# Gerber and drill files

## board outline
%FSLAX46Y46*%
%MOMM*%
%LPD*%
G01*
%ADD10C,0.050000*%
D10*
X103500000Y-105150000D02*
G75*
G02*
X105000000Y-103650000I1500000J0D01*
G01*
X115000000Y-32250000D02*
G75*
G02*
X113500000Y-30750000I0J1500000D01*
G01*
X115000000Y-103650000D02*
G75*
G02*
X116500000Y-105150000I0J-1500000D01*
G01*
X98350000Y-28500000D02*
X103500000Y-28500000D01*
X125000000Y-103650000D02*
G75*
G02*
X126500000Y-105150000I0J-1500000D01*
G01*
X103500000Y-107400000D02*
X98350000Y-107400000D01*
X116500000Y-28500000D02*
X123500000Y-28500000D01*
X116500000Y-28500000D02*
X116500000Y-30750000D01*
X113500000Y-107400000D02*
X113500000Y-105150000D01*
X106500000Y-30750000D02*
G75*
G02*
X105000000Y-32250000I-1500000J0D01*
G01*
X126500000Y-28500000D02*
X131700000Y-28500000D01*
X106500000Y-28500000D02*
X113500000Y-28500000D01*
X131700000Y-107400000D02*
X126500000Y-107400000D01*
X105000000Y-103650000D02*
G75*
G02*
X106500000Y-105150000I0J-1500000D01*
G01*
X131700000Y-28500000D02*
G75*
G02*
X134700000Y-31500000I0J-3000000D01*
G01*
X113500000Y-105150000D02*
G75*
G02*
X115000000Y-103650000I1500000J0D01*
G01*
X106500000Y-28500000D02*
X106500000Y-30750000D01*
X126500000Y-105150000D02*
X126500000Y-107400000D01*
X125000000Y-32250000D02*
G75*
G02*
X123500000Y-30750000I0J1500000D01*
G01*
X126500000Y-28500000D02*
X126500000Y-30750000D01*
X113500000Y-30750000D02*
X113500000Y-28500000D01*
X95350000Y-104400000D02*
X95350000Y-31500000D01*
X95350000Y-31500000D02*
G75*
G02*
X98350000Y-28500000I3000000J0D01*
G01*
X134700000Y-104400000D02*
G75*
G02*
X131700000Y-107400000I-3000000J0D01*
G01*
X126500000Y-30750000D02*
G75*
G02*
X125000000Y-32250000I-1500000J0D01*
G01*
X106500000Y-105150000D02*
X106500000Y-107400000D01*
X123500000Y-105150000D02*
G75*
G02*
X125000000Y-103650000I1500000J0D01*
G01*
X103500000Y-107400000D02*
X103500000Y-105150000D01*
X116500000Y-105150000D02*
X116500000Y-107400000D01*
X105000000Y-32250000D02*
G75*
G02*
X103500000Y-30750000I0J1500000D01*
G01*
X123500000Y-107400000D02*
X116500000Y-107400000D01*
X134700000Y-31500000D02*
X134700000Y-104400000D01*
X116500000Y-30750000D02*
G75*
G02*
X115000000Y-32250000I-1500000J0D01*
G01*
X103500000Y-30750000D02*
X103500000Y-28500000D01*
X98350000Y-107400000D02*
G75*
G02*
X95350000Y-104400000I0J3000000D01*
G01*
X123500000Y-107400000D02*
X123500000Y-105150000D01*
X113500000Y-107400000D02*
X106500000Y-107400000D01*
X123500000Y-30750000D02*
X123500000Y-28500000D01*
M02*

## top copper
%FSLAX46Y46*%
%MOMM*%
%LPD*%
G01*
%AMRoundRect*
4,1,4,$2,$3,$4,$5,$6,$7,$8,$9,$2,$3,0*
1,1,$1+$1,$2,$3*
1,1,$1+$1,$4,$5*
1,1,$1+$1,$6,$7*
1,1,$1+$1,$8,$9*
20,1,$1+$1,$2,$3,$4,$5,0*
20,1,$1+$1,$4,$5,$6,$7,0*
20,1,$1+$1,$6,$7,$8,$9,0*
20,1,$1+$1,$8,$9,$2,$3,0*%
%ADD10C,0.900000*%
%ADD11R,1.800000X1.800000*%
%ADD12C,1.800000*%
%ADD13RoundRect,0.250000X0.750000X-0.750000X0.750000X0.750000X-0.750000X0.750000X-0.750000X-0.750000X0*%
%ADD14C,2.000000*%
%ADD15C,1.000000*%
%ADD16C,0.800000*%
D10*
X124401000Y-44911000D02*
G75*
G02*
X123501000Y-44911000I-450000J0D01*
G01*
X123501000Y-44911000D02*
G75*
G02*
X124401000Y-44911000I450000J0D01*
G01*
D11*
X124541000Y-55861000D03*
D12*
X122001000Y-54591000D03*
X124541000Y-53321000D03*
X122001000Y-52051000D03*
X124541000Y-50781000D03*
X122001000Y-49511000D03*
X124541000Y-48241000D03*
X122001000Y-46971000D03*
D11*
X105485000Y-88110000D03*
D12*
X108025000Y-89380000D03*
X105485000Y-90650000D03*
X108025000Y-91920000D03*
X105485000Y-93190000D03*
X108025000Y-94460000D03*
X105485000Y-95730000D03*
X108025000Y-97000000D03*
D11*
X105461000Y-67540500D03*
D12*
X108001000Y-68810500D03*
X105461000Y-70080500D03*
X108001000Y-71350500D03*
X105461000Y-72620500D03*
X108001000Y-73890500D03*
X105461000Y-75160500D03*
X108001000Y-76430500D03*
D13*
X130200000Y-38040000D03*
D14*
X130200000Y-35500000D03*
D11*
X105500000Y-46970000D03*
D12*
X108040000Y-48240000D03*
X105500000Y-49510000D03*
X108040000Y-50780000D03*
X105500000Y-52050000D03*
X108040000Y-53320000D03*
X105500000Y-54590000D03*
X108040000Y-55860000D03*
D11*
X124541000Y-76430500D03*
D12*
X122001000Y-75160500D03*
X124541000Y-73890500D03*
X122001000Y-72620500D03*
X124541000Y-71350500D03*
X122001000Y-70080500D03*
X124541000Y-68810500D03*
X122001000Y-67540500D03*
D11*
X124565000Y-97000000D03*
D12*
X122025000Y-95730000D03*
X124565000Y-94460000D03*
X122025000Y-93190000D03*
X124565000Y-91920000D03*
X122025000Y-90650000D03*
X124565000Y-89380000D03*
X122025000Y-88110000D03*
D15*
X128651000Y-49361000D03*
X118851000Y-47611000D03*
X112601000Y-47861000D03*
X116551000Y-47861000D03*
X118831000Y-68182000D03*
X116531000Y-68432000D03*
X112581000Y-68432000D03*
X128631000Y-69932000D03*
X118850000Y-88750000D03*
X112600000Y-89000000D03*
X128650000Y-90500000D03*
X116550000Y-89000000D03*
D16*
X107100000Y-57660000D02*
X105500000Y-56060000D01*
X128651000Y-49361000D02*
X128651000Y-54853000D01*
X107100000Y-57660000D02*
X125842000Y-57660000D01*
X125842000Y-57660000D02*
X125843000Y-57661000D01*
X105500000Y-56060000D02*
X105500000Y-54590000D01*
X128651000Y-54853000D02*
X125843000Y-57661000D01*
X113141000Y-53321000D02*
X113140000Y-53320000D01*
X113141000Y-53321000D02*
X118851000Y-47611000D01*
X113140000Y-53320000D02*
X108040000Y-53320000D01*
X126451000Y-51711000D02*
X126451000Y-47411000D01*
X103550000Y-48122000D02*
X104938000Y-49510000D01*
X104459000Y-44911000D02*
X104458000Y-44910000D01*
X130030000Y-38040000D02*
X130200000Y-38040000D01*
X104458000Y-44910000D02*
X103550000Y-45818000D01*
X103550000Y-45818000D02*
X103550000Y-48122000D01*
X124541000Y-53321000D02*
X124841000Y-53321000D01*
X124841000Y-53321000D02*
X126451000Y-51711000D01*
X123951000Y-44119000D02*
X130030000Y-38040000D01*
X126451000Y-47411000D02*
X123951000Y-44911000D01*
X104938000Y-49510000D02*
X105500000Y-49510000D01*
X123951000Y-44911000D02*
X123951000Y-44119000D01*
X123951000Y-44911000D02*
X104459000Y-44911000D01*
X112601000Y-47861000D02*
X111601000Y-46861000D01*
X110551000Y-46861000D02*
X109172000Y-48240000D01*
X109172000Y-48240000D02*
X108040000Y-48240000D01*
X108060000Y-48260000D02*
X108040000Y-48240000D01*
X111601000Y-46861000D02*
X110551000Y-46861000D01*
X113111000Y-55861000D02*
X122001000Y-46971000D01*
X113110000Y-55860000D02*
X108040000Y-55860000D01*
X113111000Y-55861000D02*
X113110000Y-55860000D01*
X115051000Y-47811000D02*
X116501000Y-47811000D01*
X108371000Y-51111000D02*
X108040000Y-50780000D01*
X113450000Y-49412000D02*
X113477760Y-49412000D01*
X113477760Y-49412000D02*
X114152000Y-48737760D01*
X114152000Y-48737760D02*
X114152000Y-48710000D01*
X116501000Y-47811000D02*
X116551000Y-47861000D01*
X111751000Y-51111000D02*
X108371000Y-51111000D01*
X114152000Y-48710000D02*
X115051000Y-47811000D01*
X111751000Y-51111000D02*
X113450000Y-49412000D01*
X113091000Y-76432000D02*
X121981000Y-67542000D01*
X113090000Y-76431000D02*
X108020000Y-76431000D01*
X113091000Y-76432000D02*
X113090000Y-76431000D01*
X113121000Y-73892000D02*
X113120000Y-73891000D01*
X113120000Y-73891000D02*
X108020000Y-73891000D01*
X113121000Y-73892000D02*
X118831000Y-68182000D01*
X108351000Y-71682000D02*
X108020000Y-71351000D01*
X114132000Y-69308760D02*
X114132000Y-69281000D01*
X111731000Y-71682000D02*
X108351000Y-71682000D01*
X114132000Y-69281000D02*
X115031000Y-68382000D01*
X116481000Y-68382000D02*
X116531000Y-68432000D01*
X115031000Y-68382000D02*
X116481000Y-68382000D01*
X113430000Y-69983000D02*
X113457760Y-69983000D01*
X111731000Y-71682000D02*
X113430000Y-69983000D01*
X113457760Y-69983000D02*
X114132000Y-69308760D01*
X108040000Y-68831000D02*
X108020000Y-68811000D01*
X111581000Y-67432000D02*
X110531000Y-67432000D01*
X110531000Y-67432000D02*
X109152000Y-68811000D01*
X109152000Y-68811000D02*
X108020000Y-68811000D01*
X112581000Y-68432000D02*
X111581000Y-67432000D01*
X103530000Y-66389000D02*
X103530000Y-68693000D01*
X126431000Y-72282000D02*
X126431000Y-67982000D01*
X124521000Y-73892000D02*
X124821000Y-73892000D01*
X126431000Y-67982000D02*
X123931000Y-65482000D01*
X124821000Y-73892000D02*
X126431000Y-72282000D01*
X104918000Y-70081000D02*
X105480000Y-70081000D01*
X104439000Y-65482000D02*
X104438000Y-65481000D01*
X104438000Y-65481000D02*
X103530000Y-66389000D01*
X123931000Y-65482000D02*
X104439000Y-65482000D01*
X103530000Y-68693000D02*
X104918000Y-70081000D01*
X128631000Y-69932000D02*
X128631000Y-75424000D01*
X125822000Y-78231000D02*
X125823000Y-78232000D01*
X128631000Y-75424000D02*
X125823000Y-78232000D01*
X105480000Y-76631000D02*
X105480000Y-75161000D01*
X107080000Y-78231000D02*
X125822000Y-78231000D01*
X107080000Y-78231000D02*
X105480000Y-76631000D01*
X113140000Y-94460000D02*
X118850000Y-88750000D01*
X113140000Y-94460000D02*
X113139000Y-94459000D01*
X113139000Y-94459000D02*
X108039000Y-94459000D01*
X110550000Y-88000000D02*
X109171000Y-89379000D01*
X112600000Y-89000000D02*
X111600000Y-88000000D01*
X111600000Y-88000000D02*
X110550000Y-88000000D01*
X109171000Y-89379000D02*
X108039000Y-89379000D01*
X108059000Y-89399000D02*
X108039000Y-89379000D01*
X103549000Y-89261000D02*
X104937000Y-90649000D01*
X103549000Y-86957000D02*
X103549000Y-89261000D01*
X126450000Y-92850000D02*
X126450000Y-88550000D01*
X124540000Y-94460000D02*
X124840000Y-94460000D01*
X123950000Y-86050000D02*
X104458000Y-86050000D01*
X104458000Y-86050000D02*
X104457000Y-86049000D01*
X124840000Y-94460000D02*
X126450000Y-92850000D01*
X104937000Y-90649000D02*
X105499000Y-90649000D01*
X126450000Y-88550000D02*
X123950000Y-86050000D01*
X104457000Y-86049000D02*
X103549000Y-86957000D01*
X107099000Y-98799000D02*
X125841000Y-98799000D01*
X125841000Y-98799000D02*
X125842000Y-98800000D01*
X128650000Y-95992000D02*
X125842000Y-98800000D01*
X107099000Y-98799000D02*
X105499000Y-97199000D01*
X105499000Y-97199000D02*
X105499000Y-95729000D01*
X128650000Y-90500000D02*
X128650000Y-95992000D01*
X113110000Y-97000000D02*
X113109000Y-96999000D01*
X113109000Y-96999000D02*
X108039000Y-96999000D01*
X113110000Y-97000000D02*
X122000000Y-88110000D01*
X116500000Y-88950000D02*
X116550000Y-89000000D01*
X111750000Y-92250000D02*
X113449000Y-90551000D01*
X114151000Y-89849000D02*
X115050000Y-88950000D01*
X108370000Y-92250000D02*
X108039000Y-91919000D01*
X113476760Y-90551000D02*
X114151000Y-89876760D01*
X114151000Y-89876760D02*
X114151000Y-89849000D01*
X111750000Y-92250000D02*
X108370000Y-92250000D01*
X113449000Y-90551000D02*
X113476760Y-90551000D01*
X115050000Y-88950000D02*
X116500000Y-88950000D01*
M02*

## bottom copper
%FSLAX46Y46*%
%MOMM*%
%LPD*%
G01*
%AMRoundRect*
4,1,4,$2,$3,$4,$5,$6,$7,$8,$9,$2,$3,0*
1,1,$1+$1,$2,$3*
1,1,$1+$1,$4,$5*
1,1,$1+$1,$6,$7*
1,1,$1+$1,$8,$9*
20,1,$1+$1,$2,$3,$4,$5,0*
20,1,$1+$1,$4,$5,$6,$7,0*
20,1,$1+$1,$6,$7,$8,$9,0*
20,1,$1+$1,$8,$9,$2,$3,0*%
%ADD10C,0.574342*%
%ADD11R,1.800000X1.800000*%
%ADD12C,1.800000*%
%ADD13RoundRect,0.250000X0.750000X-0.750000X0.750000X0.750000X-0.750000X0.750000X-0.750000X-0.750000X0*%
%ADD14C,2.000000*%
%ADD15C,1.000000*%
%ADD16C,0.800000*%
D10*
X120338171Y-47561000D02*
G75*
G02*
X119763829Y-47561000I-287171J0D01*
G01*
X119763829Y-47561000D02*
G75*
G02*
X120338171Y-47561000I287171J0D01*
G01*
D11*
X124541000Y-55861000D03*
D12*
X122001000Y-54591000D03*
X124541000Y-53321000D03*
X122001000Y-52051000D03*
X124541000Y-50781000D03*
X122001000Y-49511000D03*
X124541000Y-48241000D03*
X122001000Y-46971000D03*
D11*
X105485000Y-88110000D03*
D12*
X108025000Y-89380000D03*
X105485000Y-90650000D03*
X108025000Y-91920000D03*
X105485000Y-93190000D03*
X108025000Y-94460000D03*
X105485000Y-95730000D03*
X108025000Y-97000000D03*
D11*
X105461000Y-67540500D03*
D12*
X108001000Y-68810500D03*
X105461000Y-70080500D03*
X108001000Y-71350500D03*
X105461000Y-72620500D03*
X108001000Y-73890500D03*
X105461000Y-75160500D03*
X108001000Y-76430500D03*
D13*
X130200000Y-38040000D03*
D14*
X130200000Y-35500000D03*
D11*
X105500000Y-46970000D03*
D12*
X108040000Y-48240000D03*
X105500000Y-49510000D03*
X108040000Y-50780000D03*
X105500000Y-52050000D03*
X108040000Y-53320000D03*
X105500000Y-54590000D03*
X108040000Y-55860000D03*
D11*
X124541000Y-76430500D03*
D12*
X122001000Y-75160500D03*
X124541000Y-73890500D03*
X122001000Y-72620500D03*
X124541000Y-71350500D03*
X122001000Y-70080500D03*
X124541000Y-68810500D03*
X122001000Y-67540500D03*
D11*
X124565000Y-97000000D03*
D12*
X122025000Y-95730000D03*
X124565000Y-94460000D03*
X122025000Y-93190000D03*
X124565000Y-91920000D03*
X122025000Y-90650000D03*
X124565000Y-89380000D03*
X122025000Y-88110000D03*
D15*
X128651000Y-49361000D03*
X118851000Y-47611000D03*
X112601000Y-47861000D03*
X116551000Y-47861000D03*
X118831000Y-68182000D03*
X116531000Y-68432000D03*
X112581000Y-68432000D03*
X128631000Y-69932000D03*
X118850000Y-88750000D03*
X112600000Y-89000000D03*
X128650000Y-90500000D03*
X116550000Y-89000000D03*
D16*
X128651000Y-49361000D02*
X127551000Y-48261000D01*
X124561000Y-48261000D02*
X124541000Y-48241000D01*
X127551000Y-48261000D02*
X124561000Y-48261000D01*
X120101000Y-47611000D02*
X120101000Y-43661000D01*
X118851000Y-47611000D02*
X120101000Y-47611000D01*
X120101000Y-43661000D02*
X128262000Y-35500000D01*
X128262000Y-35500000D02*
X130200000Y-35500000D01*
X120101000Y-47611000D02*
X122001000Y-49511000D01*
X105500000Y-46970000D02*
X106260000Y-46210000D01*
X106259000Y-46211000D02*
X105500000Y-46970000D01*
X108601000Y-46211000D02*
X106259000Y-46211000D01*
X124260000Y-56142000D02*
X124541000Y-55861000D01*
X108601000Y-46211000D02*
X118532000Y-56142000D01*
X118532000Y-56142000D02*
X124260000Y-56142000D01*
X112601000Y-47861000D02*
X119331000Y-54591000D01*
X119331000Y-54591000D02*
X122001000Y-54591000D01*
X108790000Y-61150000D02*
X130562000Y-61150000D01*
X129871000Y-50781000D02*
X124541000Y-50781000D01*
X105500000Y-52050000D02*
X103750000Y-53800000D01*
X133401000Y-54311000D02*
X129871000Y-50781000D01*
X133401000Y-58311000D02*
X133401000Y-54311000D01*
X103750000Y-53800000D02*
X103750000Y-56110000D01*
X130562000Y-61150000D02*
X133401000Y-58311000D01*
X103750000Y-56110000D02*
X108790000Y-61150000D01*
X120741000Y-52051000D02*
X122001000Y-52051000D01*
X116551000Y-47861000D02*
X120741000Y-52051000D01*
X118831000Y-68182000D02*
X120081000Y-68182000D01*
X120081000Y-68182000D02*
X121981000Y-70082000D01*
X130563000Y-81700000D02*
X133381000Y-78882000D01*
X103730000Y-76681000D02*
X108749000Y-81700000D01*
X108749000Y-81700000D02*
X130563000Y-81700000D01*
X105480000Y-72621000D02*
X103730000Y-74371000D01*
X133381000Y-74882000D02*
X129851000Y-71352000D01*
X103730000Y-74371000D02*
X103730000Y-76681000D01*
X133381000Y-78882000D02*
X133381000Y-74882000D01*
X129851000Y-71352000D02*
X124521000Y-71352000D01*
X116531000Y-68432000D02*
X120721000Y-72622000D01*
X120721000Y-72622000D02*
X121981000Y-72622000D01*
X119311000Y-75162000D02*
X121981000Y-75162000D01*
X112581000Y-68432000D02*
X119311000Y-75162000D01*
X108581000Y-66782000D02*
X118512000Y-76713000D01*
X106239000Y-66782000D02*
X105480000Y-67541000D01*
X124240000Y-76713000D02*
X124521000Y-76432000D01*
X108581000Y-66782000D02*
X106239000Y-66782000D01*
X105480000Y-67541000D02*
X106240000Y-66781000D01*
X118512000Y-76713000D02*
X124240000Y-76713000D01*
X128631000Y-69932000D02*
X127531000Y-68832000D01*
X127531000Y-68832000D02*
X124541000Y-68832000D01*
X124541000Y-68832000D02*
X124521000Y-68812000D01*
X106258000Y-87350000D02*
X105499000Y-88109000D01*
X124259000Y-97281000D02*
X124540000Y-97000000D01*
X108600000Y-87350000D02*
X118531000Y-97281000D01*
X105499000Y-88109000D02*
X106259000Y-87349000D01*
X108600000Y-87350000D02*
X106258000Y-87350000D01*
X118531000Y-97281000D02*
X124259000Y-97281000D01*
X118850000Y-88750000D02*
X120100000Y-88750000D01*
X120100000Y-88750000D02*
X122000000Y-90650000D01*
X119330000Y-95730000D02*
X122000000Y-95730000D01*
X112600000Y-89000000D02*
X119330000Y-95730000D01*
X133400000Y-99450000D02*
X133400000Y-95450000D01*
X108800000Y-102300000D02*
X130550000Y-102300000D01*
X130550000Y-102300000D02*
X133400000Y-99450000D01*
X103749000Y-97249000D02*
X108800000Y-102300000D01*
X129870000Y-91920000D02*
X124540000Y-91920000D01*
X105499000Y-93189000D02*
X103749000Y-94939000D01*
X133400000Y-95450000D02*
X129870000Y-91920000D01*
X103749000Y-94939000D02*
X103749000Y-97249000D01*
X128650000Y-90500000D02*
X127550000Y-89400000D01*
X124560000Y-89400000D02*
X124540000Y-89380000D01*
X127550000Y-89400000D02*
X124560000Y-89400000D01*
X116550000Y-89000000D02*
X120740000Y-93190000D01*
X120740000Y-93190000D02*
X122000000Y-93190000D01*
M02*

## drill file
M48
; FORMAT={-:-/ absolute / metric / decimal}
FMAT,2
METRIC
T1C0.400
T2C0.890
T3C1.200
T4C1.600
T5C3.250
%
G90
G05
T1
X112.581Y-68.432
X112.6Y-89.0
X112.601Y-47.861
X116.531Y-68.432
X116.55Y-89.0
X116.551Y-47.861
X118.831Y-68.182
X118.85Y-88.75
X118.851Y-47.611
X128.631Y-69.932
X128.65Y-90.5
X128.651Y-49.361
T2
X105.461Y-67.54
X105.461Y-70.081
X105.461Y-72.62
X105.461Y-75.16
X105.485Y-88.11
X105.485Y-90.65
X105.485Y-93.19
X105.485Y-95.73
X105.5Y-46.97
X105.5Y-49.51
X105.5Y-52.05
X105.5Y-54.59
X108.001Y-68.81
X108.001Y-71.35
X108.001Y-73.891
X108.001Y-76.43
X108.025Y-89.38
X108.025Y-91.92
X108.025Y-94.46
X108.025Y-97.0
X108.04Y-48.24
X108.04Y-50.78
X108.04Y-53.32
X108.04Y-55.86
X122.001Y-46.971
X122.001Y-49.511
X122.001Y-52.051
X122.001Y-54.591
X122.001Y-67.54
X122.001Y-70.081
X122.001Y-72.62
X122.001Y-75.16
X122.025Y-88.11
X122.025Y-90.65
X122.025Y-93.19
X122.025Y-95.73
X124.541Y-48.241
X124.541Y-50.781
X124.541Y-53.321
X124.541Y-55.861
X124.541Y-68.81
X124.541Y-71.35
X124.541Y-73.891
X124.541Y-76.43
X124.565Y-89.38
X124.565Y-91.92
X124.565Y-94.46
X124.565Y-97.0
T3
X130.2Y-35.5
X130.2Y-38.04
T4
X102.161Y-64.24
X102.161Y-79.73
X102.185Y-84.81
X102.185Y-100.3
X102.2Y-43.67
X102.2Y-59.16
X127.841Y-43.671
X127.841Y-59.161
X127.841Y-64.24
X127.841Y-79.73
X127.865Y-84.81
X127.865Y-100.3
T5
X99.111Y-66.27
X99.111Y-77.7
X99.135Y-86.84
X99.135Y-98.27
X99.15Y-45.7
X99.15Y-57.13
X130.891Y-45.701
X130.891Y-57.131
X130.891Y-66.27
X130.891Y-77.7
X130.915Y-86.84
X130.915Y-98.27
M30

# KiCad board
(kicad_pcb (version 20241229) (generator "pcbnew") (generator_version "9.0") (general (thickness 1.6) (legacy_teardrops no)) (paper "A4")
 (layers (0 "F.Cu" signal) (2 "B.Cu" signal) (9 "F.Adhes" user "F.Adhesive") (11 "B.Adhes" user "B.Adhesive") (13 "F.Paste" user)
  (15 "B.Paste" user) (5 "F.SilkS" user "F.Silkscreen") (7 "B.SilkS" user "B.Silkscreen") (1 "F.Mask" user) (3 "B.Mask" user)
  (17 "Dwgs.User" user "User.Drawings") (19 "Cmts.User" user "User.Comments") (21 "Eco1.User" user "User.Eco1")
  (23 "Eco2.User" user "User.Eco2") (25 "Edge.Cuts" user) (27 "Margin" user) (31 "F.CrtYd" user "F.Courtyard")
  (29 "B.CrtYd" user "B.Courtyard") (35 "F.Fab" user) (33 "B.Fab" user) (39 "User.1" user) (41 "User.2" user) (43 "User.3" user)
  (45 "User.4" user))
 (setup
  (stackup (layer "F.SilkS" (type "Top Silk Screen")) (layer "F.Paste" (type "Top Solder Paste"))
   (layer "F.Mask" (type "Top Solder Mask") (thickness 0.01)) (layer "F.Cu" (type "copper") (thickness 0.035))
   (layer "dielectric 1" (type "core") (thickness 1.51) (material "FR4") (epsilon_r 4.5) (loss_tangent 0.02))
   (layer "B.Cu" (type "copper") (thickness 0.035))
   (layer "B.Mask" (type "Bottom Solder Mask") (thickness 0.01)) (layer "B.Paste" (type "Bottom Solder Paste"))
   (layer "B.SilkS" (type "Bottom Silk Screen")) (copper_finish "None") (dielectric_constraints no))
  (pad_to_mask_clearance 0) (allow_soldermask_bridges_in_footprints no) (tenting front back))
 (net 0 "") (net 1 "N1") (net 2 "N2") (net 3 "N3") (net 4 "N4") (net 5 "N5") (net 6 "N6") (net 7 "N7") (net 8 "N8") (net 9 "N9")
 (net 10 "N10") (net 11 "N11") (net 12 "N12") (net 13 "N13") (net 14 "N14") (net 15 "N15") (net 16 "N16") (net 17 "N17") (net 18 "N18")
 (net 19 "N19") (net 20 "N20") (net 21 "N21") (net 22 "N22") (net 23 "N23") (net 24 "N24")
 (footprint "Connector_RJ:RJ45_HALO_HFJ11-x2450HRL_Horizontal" (layer "F.Cu") (at 124.541 55.861 90)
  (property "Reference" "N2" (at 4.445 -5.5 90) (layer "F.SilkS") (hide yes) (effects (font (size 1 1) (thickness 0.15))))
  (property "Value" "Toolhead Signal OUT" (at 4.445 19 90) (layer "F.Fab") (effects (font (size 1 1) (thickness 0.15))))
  (pad "" np_thru_hole circle (at -3.3 3.3 90) (size 3 3) (drill 1.6) (layers "*.Mask"))
  (pad "" np_thru_hole circle (at -1.27 6.35 90) (size 3.25 3.25) (drill 3.25) (layers "*.Cu" "*.Mask"))
  (pad "" np_thru_hole circle (at 10.16 6.35 90) (size 3.25 3.25) (drill 3.25) (layers "*.Cu" "*.Mask"))
  (pad "" np_thru_hole circle (at 12.19 3.3 90) (size 3 3) (drill 1.6) (layers "*.Mask"))
  (pad "1" thru_hole rect (at 0 0 90) (size 1.8 1.8) (drill 0.89) (layers "*.Cu" "*.Mask") (remove_unused_layers no) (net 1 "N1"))
  (pad "2" thru_hole circle (at 1.27 -2.54 90) (size 1.8 1.8) (drill 0.89) (layers "*.Cu" "*.Mask") (remove_unused_layers no) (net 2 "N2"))
  (pad "3" thru_hole circle (at 2.54 0 90) (size 1.8 1.8) (drill 0.89) (layers "*.Cu" "*.Mask") (remove_unused_layers no) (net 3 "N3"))
  (pad "4" thru_hole circle (at 3.81 -2.54 90) (size 1.8 1.8) (drill 0.89) (layers "*.Cu" "*.Mask") (remove_unused_layers no) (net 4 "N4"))
  (pad "5" thru_hole circle (at 5.08 0 90) (size 1.8 1.8) (drill 0.89) (layers "*.Cu" "*.Mask") (remove_unused_layers no) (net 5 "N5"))
  (pad "6" thru_hole circle (at 6.35 -2.54 90) (size 1.8 1.8) (drill 0.89) (layers "*.Cu" "*.Mask") (remove_unused_layers no) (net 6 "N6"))
  (pad "7" thru_hole circle (at 7.62 0 90) (size 1.8 1.8) (drill 0.89) (layers "*.Cu" "*.Mask") (remove_unused_layers no) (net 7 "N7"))
  (pad "8" thru_hole circle (at 8.89 -2.54 90) (size 1.8 1.8) (drill 0.89) (layers "*.Cu" "*.Mask") (remove_unused_layers no) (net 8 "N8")))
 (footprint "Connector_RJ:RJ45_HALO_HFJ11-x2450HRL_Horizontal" (layer "F.Cu") (at 105.485 88.11 -90)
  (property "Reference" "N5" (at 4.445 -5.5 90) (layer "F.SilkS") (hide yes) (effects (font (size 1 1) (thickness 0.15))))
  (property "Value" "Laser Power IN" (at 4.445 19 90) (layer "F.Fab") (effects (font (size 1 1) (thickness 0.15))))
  (pad "" np_thru_hole circle (at -3.3 3.3 270) (size 3 3) (drill 1.6) (layers "*.Mask"))
  (pad "" np_thru_hole circle (at -1.27 6.35 270) (size 3.25 3.25) (drill 3.25) (layers "*.Cu" "*.Mask"))
  (pad "" np_thru_hole circle (at 10.16 6.35 270) (size 3.25 3.25) (drill 3.25) (layers "*.Cu" "*.Mask"))
  (pad "" np_thru_hole circle (at 12.19 3.3 270) (size 3 3) (drill 1.6) (layers "*.Mask"))
  (pad "1" thru_hole rect (at 0 0 270) (size 1.8 1.8) (drill 0.89) (layers "*.Cu" "*.Mask") (remove_unused_layers no) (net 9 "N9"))
  (pad "2" thru_hole circle (at 1.27 -2.54 270) (size 1.8 1.8) (drill 0.89) (layers "*.Cu" "*.Mask") (remove_unused_layers no)
   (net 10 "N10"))
  (pad "3" thru_hole circle (at 2.54 0 270) (size 1.8 1.8) (drill 0.89) (layers "*.Cu" "*.Mask") (remove_unused_layers no) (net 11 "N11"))
  (pad "4" thru_hole circle (at 3.81 -2.54 270) (size 1.8 1.8) (drill 0.89) (layers "*.Cu" "*.Mask") (remove_unused_layers no)
   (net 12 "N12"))
  (pad "5" thru_hole circle (at 5.08 0 270) (size 1.8 1.8) (drill 0.89) (layers "*.Cu" "*.Mask") (remove_unused_layers no) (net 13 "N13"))
  (pad "6" thru_hole circle (at 6.35 -2.54 270) (size 1.8 1.8) (drill 0.89) (layers "*.Cu" "*.Mask") (remove_unused_layers no)
   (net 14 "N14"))
  (pad "7" thru_hole circle (at 7.62 0 270) (size 1.8 1.8) (drill 0.89) (layers "*.Cu" "*.Mask") (remove_unused_layers no) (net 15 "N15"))
  (pad "8" thru_hole circle (at 8.89 -2.54 270) (size 1.8 1.8) (drill 0.89) (layers "*.Cu" "*.Mask") (remove_unused_layers no)
   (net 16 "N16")))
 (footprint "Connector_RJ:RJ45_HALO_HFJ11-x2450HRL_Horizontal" (layer "F.Cu") (at 105.461 67.5405 -90)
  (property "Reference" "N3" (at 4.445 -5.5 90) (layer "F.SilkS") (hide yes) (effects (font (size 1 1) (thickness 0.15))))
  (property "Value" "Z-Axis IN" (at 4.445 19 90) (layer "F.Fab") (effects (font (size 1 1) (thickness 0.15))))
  (pad "" np_thru_hole circle (at -3.3 3.3 270) (size 3 3) (drill 1.6) (layers "*.Mask"))
  (pad "" np_thru_hole circle (at -1.27 6.35 270) (size 3.25 3.25) (drill 3.25) (layers "*.Cu" "*.Mask"))
  (pad "" np_thru_hole circle (at 10.16 6.35 270) (size 3.25 3.25) (drill 3.25) (layers "*.Cu" "*.Mask"))
  (pad "" np_thru_hole circle (at 12.19 3.3 270) (size 3 3) (drill 1.6) (layers "*.Mask"))
  (pad "1" thru_hole rect (at 0 0 270) (size 1.8 1.8) (drill 0.89) (layers "*.Cu" "*.Mask") (remove_unused_layers no) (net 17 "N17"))
  (pad "2" thru_hole circle (at 1.27 -2.54 270) (size 1.8 1.8) (drill 0.89) (layers "*.Cu" "*.Mask") (remove_unused_layers no)
   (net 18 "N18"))
  (pad "3" thru_hole circle (at 2.54 0 270) (size 1.8 1.8) (drill 0.89) (layers "*.Cu" "*.Mask") (remove_unused_layers no) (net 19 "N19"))
  (pad "4" thru_hole circle (at 3.81 -2.54 270) (size 1.8 1.8) (drill 0.89) (layers "*.Cu" "*.Mask") (remove_unused_layers no)
   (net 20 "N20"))
  (pad "5" thru_hole circle (at 5.08 0 270) (size 1.8 1.8) (drill 0.89) (layers "*.Cu" "*.Mask") (remove_unused_layers no) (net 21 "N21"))
  (pad "6" thru_hole circle (at 6.35 -2.54 270) (size 1.8 1.8) (drill 0.89) (layers "*.Cu" "*.Mask") (remove_unused_layers no)
   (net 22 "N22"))
  (pad "7" thru_hole circle (at 7.62 0 270) (size 1.8 1.8) (drill 0.89) (layers "*.Cu" "*.Mask") (remove_unused_layers no) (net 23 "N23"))
  (pad "8" thru_hole circle (at 8.89 -2.54 270) (size 1.8 1.8) (drill 0.89) (layers "*.Cu" "*.Mask") (remove_unused_layers no)
   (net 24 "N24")))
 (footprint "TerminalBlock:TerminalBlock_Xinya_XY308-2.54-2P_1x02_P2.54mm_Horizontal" (layer "F.Cu") (at 130.2 38.04 90)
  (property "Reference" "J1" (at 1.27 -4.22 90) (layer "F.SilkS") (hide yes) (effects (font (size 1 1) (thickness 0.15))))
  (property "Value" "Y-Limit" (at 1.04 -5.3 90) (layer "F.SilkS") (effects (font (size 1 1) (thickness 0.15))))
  (pad "1" thru_hole roundrect (at 0 0 90) (size 2 2) (drill 1.2) (layers "*.Cu" "*.Mask") (remove_unused_layers no)
   (roundrect_rratio 0.125) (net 3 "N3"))
  (pad "2" thru_hole circle (at 2.54 0 90) (size 2 2) (drill 1.2) (layers "*.Cu" "*.Mask") (remove_unused_layers no) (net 6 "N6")))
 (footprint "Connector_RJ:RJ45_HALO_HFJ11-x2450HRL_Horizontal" (layer "F.Cu") (at 105.5 46.97 -90)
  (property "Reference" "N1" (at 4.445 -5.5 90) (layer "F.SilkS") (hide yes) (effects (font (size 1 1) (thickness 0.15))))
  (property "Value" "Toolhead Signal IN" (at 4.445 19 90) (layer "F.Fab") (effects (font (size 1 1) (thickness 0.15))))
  (pad "" np_thru_hole circle (at -3.3 3.3 270) (size 3 3) (drill 1.6) (layers "*.Mask"))
  (pad "" np_thru_hole circle (at -1.27 6.35 270) (size 3.25 3.25) (drill 3.25) (layers "*.Cu" "*.Mask"))
  (pad "" np_thru_hole circle (at 10.16 6.35 270) (size 3.25 3.25) (drill 3.25) (layers "*.Cu" "*.Mask"))
  (pad "" np_thru_hole circle (at 12.19 3.3 270) (size 3 3) (drill 1.6) (layers "*.Mask"))
  (pad "1" thru_hole rect (at 0 0 270) (size 1.8 1.8) (drill 0.89) (layers "*.Cu" "*.Mask") (remove_unused_layers no) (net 1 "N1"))
  (pad "2" thru_hole circle (at 1.27 -2.54 270) (size 1.8 1.8) (drill 0.89) (layers "*.Cu" "*.Mask") (remove_unused_layers no) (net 2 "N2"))
  (pad "3" thru_hole circle (at 2.54 0 270) (size 1.8 1.8) (drill 0.89) (layers "*.Cu" "*.Mask") (remove_unused_layers no) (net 3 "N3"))
  (pad "4" thru_hole circle (at 3.81 -2.54 270) (size 1.8 1.8) (drill 0.89) (layers "*.Cu" "*.Mask") (remove_unused_layers no) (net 4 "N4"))
  (pad "5" thru_hole circle (at 5.08 0 270) (size 1.8 1.8) (drill 0.89) (layers "*.Cu" "*.Mask") (remove_unused_layers no) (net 5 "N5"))
  (pad "6" thru_hole circle (at 6.35 -2.54 270) (size 1.8 1.8) (drill 0.89) (layers "*.Cu" "*.Mask") (remove_unused_layers no) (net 6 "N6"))
  (pad "7" thru_hole circle (at 7.62 0 270) (size 1.8 1.8) (drill 0.89) (layers "*.Cu" "*.Mask") (remove_unused_layers no) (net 7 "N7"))
  (pad "8" thru_hole circle (at 8.89 -2.54 270) (size 1.8 1.8) (drill 0.89) (layers "*.Cu" "*.Mask") (remove_unused_layers no) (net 8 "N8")))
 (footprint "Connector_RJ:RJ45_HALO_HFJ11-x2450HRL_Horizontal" (layer "F.Cu") (at 124.541 76.4305 90)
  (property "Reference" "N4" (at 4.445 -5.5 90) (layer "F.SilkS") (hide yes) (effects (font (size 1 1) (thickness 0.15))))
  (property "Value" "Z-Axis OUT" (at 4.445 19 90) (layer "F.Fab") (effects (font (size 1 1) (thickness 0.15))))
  (pad "" np_thru_hole circle (at -3.3 3.3 90) (size 3 3) (drill 1.6) (layers "*.Mask"))
  (pad "" np_thru_hole circle (at -1.27 6.35 90) (size 3.25 3.25) (drill 3.25) (layers "*.Cu" "*.Mask"))
  (pad "" np_thru_hole circle (at 10.16 6.35 90) (size 3.25 3.25) (drill 3.25) (layers "*.Cu" "*.Mask"))
  (pad "" np_thru_hole circle (at 12.19 3.3 90) (size 3 3) (drill 1.6) (layers "*.Mask"))
  (pad "1" thru_hole rect (at 0 0 90) (size 1.8 1.8) (drill 0.89) (layers "*.Cu" "*.Mask") (remove_unused_layers no) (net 17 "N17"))
  (pad "2" thru_hole circle (at 1.27 -2.54 90) (size 1.8 1.8) (drill 0.89) (layers "*.Cu" "*.Mask") (remove_unused_layers no) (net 18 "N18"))
  (pad "3" thru_hole circle (at 2.54 0 90) (size 1.8 1.8) (drill 0.89) (layers "*.Cu" "*.Mask") (remove_unused_layers no) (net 19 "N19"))
  (pad "4" thru_hole circle (at 3.81 -2.54 90) (size 1.8 1.8) (drill 0.89) (layers "*.Cu" "*.Mask") (remove_unused_layers no) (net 20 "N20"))
  (pad "5" thru_hole circle (at 5.08 0 90) (size 1.8 1.8) (drill 0.89) (layers "*.Cu" "*.Mask") (remove_unused_layers no) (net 21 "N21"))
  (pad "6" thru_hole circle (at 6.35 -2.54 90) (size 1.8 1.8) (drill 0.89) (layers "*.Cu" "*.Mask") (remove_unused_layers no) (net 22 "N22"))
  (pad "7" thru_hole circle (at 7.62 0 90) (size 1.8 1.8) (drill 0.89) (layers "*.Cu" "*.Mask") (remove_unused_layers no) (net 23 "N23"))
  (pad "8" thru_hole circle (at 8.89 -2.54 90) (size 1.8 1.8) (drill 0.89) (layers "*.Cu" "*.Mask") (remove_unused_layers no) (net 24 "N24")))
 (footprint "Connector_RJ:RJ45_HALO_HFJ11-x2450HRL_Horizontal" (layer "F.Cu") (at 124.565 97 90)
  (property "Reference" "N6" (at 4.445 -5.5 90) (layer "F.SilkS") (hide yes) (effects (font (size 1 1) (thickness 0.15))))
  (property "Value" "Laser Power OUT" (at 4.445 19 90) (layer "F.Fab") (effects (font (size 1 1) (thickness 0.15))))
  (pad "" np_thru_hole circle (at -3.3 3.3 90) (size 3 3) (drill 1.6) (layers "*.Mask"))
  (pad "" np_thru_hole circle (at -1.27 6.35 90) (size 3.25 3.25) (drill 3.25) (layers "*.Cu" "*.Mask"))
  (pad "" np_thru_hole circle (at 10.16 6.35 90) (size 3.25 3.25) (drill 3.25) (layers "*.Cu" "*.Mask"))
  (pad "" np_thru_hole circle (at 12.19 3.3 90) (size 3 3) (drill 1.6) (layers "*.Mask"))
  (pad "1" thru_hole rect (at 0 0 90) (size 1.8 1.8) (drill 0.89) (layers "*.Cu" "*.Mask") (remove_unused_layers no) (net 9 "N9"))
  (pad "2" thru_hole circle (at 1.27 -2.54 90) (size 1.8 1.8) (drill 0.89) (layers "*.Cu" "*.Mask") (remove_unused_layers no) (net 10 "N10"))
  (pad "3" thru_hole circle (at 2.54 0 90) (size 1.8 1.8) (drill 0.89) (layers "*.Cu" "*.Mask") (remove_unused_layers no) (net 11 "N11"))
  (pad "4" thru_hole circle (at 3.81 -2.54 90) (size 1.8 1.8) (drill 0.89) (layers "*.Cu" "*.Mask") (remove_unused_layers no) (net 12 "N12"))
  (pad "5" thru_hole circle (at 5.08 0 90) (size 1.8 1.8) (drill 0.89) (layers "*.Cu" "*.Mask") (remove_unused_layers no) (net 13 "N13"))
  (pad "6" thru_hole circle (at 6.35 -2.54 90) (size 1.8 1.8) (drill 0.89) (layers "*.Cu" "*.Mask") (remove_unused_layers no) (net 14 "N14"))
  (pad "7" thru_hole circle (at 7.62 0 90) (size 1.8 1.8) (drill 0.89) (layers "*.Cu" "*.Mask") (remove_unused_layers no) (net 15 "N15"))
  (pad "8" thru_hole circle (at 8.89 -2.54 90) (size 1.8 1.8) (drill 0.89) (layers "*.Cu" "*.Mask") (remove_unused_layers no) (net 16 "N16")))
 (gr_circle (center 123.951 44.911) (end 124.751 44.911) (stroke (width 0.2) (type solid)) (fill yes) (layer "F.Cu") (net 3))
 (gr_circle (center 120.051 47.561) (end 120.501 47.411) (stroke (width 0.2) (type solid)) (fill yes) (layer "B.Cu") (net 6))
 (gr_arc (start 103.5 105.15) (mid 103.93934 104.08934) (end 105 103.65) (stroke (width 0.05) (type default)) (layer "Edge.Cuts"))
 (gr_arc (start 115 32.25) (mid 113.93934 31.81066) (end 113.5 30.75) (stroke (width 0.05) (type default)) (layer "Edge.Cuts"))
 (gr_arc (start 115 103.65) (mid 116.06066 104.08934) (end 116.5 105.15) (stroke (width 0.05) (type default)) (layer "Edge.Cuts"))
 (gr_line (start 98.35 28.5) (end 103.5 28.5) (stroke (width 0.05) (type default)) (layer "Edge.Cuts"))
 (gr_arc (start 125 103.65) (mid 126.06066 104.08934) (end 126.5 105.15) (stroke (width 0.05) (type default)) (layer "Edge.Cuts"))
 (gr_line (start 103.5 107.4) (end 98.35 107.4) (stroke (width 0.05) (type default)) (layer "Edge.Cuts"))
 (gr_line (start 116.5 28.5) (end 123.5 28.5) (stroke (width 0.05) (type default)) (layer "Edge.Cuts"))
 (gr_line (start 116.5 28.5) (end 116.5 30.75) (stroke (width 0.05) (type solid)) (layer "Edge.Cuts"))
 (gr_line (start 113.5 107.4) (end 113.5 105.15) (stroke (width 0.05) (type solid)) (layer "Edge.Cuts"))
 (gr_arc (start 106.5 30.75) (mid 106.06066 31.81066) (end 105 32.25) (stroke (width 0.05) (type default)) (layer "Edge.Cuts"))
 (gr_line (start 126.5 28.5) (end 131.7 28.5) (stroke (width 0.05) (type default)) (layer "Edge.Cuts"))
 (gr_line (start 106.5 28.5) (end 113.5 28.5) (stroke (width 0.05) (type default)) (layer "Edge.Cuts"))
 (gr_line (start 131.7 107.4) (end 126.5 107.4) (stroke (width 0.05) (type default)) (layer "Edge.Cuts"))
 (gr_arc (start 105 103.65) (mid 106.06066 104.08934) (end 106.5 105.15) (stroke (width 0.05) (type default)) (layer "Edge.Cuts"))
 (gr_arc (start 131.7 28.5) (mid 133.82132 29.37868) (end 134.7 31.5) (stroke (width 0.05) (type default)) (layer "Edge.Cuts"))
 (gr_arc (start 113.5 105.15) (mid 113.93934 104.08934) (end 115 103.65) (stroke (width 0.05) (type default)) (layer "Edge.Cuts"))
 (gr_line (start 106.5 28.5) (end 106.5 30.75) (stroke (width 0.05) (type solid)) (layer "Edge.Cuts"))
 (gr_line (start 126.5 105.15) (end 126.5 107.4) (stroke (width 0.05) (type solid)) (layer "Edge.Cuts"))
 (gr_arc (start 125 32.25) (mid 123.93934 31.81066) (end 123.5 30.75) (stroke (width 0.05) (type default)) (layer "Edge.Cuts"))
 (gr_line (start 126.5 28.5) (end 126.5 30.75) (stroke (width 0.05) (type solid)) (layer "Edge.Cuts"))
 (gr_line (start 113.5 30.75) (end 113.5 28.5) (stroke (width 0.05) (type solid)) (layer "Edge.Cuts"))
 (gr_line (start 95.35 104.4) (end 95.35 31.5) (stroke (width 0.05) (type default)) (layer "Edge.Cuts"))
 (gr_arc (start 95.35 31.5) (mid 96.22868 29.37868) (end 98.35 28.5) (stroke (width 0.05) (type default)) (layer "Edge.Cuts"))
 (gr_arc (start 134.7 104.4) (mid 133.82132 106.52132) (end 131.7 107.4) (stroke (width 0.05) (type default)) (layer "Edge.Cuts"))
 (gr_arc (start 126.5 30.75) (mid 126.06066 31.81066) (end 125 32.25) (stroke (width 0.05) (type default)) (layer "Edge.Cuts"))
 (gr_line (start 106.5 105.15) (end 106.5 107.4) (stroke (width 0.05) (type solid)) (layer "Edge.Cuts"))
 (gr_arc (start 123.5 105.15) (mid 123.93934 104.08934) (end 125 103.65) (stroke (width 0.05) (type default)) (layer "Edge.Cuts"))
 (gr_line (start 103.5 107.4) (end 103.5 105.15) (stroke (width 0.05) (type solid)) (layer "Edge.Cuts"))
 (gr_line (start 116.5 105.15) (end 116.5 107.4) (stroke (width 0.05) (type solid)) (layer "Edge.Cuts"))
 (gr_arc (start 105 32.25) (mid 103.93934 31.81066) (end 103.5 30.75) (stroke (width 0.05) (type default)) (layer "Edge.Cuts"))
 (gr_line (start 123.5 107.4) (end 116.5 107.4) (stroke (width 0.05) (type default)) (layer "Edge.Cuts"))
 (gr_line (start 134.7 31.5) (end 134.7 104.4) (stroke (width 0.05) (type default)) (layer "Edge.Cuts"))
 (gr_arc (start 116.5 30.75) (mid 116.06066 31.81066) (end 115 32.25) (stroke (width 0.05) (type default)) (layer "Edge.Cuts"))
 (gr_line (start 103.5 30.75) (end 103.5 28.5) (stroke (width 0.05) (type solid)) (layer "Edge.Cuts"))
 (gr_arc (start 98.35 107.4) (mid 96.22868 106.52132) (end 95.35 104.4) (stroke (width 0.05) (type default)) (layer "Edge.Cuts"))
 (gr_line (start 123.5 107.4) (end 123.5 105.15) (stroke (width 0.05) (type solid)) (layer "Edge.Cuts"))
 (gr_line (start 113.5 107.4) (end 106.5 107.4) (stroke (width 0.05) (type default)) (layer "Edge.Cuts"))
 (gr_line (start 123.5 30.75) (end 123.5 28.5) (stroke (width 0.05) (type solid)) (layer "Edge.Cuts"))
 (segment (start 107.1 57.66) (end 105.5 56.06) (width 0.8) (layer "F.Cu") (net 7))
 (segment (start 128.651 49.361) (end 128.651 54.853) (width 0.8) (layer "F.Cu") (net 7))
 (segment (start 107.1 57.66) (end 125.842 57.66) (width 0.8) (layer "F.Cu") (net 7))
 (segment (start 125.842 57.66) (end 125.843 57.661) (width 0.8) (layer "F.Cu") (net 7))
 (segment (start 105.5 56.06) (end 105.5 54.59) (width 0.8) (layer "F.Cu") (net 7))
 (segment (start 128.651 54.853) (end 125.843 57.661) (width 0.8) (layer "F.Cu") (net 7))
 (via (at 128.651 49.361) (size 1) (drill 0.4) (layers "F.Cu" "B.Cu") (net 7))
 (segment (start 128.651 49.361) (end 127.551 48.261) (width 0.8) (layer "B.Cu") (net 7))
 (segment (start 124.561 48.261) (end 124.541 48.241) (width 0.8) (layer "B.Cu") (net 7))
 (segment (start 127.551 48.261) (end 124.561 48.261) (width 0.8) (layer "B.Cu") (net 7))
 (segment (start 113.141 53.321) (end 113.14 53.32) (width 0.8) (layer "F.Cu") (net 6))
 (segment (start 113.141 53.321) (end 118.851 47.611) (width 0.8) (layer "F.Cu") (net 6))
 (segment (start 113.14 53.32) (end 108.04 53.32) (width 0.8) (layer "F.Cu") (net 6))
 (via (at 118.851 47.611) (size 1) (drill 0.4) (layers "F.Cu" "B.Cu") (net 6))
 (segment (start 120.101 47.611) (end 120.101 43.661) (width 0.8) (layer "B.Cu") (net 6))
 (segment (start 118.851 47.611) (end 120.101 47.611) (width 0.8) (layer "B.Cu") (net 6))
 (segment (start 120.101 43.661) (end 128.262 35.5) (width 0.8) (layer "B.Cu") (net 6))
 (segment (start 128.262 35.5) (end 130.2 35.5) (width 0.8) (layer "B.Cu") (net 6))
 (segment (start 120.101 47.611) (end 122.001 49.511) (width 0.8) (layer "B.Cu") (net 6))
 (segment (start 126.451 51.711) (end 126.451 47.411) (width 0.8) (layer "F.Cu") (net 3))
 (segment (start 103.55 48.122) (end 104.938 49.51) (width 0.8) (layer "F.Cu") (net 3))
 (segment (start 104.459 44.911) (end 104.458 44.91) (width 0.8) (layer "F.Cu") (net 3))
 (segment (start 130.03 38.04) (end 130.2 38.04) (width 0.8) (layer "F.Cu") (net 3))
 (segment (start 104.458 44.91) (end 103.55 45.818) (width 0.8) (layer "F.Cu") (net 3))
 (segment (start 103.55 45.818) (end 103.55 48.122) (width 0.8) (layer "F.Cu") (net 3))
 (segment (start 124.541 53.321) (end 124.841 53.321) (width 0.8) (layer "F.Cu") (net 3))
 (segment (start 124.841 53.321) (end 126.451 51.711) (width 0.8) (layer "F.Cu") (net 3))
 (segment (start 123.951 44.119) (end 130.03 38.04) (width 0.8) (layer "F.Cu") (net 3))
 (segment (start 126.451 47.411) (end 123.951 44.911) (width 0.8) (layer "F.Cu") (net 3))
 (segment (start 104.938 49.51) (end 105.5 49.51) (width 0.8) (layer "F.Cu") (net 3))
 (segment (start 123.951 44.911) (end 123.951 44.119) (width 0.8) (layer "F.Cu") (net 3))
 (segment (start 123.951 44.911) (end 104.459 44.911) (width 0.8) (layer "F.Cu") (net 3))
 (segment (start 105.5 46.97) (end 106.26 46.21) (width 0.8) (layer "B.Cu") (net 1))
 (segment (start 106.259 46.211) (end 105.5 46.97) (width 0.8) (layer "B.Cu") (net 1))
 (segment (start 108.601 46.211) (end 106.259 46.211) (width 0.8) (layer "B.Cu") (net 1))
 (segment (start 124.26 56.142) (end 124.541 55.861) (width 0.8) (layer "B.Cu") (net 1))
 (segment (start 108.601 46.211) (end 118.532 56.142) (width 0.8) (layer "B.Cu") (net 1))
 (segment (start 118.532 56.142) (end 124.26 56.142) (width 0.8) (layer "B.Cu") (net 1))
 (segment (start 112.601 47.861) (end 111.601 46.861) (width 0.8) (layer "F.Cu") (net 2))
 (segment (start 110.551 46.861) (end 109.172 48.24) (width 0.8) (layer "F.Cu") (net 2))
 (segment (start 109.172 48.24) (end 108.04 48.24) (width 0.8) (layer "F.Cu") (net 2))
 (segment (start 108.06 48.26) (end 108.04 48.24) (width 0.8) (layer "F.Cu") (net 2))
 (segment (start 111.601 46.861) (end 110.551 46.861) (width 0.8) (layer "F.Cu") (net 2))
 (via (at 112.601 47.861) (size 1) (drill 0.4) (layers "F.Cu" "B.Cu") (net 2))
 (segment (start 112.601 47.861) (end 119.331 54.591) (width 0.8) (layer "B.Cu") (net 2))
 (segment (start 119.331 54.591) (end 122.001 54.591) (width 0.8) (layer "B.Cu") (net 2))
 (segment (start 108.79 61.15) (end 130.562 61.15) (width 0.8) (layer "B.Cu") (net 5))
 (segment (start 129.871 50.781) (end 124.541 50.781) (width 0.8) (layer "B.Cu") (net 5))
 (segment (start 105.5 52.05) (end 103.75 53.8) (width 0.8) (layer "B.Cu") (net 5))
 (segment (start 133.401 54.311) (end 129.871 50.781) (width 0.8) (layer "B.Cu") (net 5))
 (segment (start 133.401 58.311) (end 133.401 54.311) (width 0.8) (layer "B.Cu") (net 5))
 (segment (start 103.75 53.8) (end 103.75 56.11) (width 0.8) (layer "B.Cu") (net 5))
 (segment (start 130.562 61.15) (end 133.401 58.311) (width 0.8) (layer "B.Cu") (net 5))
 (segment (start 103.75 56.11) (end 108.79 61.15) (width 0.8) (layer "B.Cu") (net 5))
 (segment (start 113.111 55.861) (end 122.001 46.971) (width 0.8) (layer "F.Cu") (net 8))
 (segment (start 113.11 55.86) (end 108.04 55.86) (width 0.8) (layer "F.Cu") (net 8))
 (segment (start 113.111 55.861) (end 113.11 55.86) (width 0.8) (layer "F.Cu") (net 8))
 (segment (start 115.051 47.811) (end 116.501 47.811) (width 0.8) (layer "F.Cu") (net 4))
 (segment (start 108.371 51.111) (end 108.04 50.78) (width 0.8) (layer "F.Cu") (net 4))
 (segment (start 113.45 49.412) (end 113.47776 49.412) (width 0.8) (layer "F.Cu") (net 4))
 (segment (start 113.47776 49.412) (end 114.152 48.73776) (width 0.8) (layer "F.Cu") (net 4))
 (segment (start 114.152 48.73776) (end 114.152 48.71) (width 0.8) (layer "F.Cu") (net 4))
 (segment (start 116.501 47.811) (end 116.551 47.861) (width 0.8) (layer "F.Cu") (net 4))
 (segment (start 111.751 51.111) (end 108.371 51.111) (width 0.8) (layer "F.Cu") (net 4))
 (segment (start 114.152 48.71) (end 115.051 47.811) (width 0.8) (layer "F.Cu") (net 4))
 (segment (start 111.751 51.111) (end 113.45 49.412) (width 0.8) (layer "F.Cu") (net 4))
 (via (at 116.551 47.861) (size 1) (drill 0.4) (layers "F.Cu" "B.Cu") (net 4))
 (segment (start 120.741 52.051) (end 122.001 52.051) (width 0.8) (layer "B.Cu") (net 4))
 (segment (start 116.551 47.861) (end 120.741 52.051) (width 0.8) (layer "B.Cu") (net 4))
 (segment (start 113.091 76.432) (end 121.981 67.542) (width 0.8) (layer "F.Cu") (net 24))
 (segment (start 113.09 76.431) (end 108.02 76.431) (width 0.8) (layer "F.Cu") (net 24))
 (segment (start 113.091 76.432) (end 113.09 76.431) (width 0.8) (layer "F.Cu") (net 24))
 (segment (start 113.121 73.892) (end 113.12 73.891) (width 0.8) (layer "F.Cu") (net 22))
 (segment (start 113.12 73.891) (end 108.02 73.891) (width 0.8) (layer "F.Cu") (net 22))
 (segment (start 113.121 73.892) (end 118.831 68.182) (width 0.8) (layer "F.Cu") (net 22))
 (via (at 118.831 68.182) (size 1) (drill 0.4) (layers "F.Cu" "B.Cu") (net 22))
 (segment (start 118.831 68.182) (end 120.081 68.182) (width 0.8) (layer "B.Cu") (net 22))
 (segment (start 120.081 68.182) (end 121.981 70.082) (width 0.8) (layer "B.Cu") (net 22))
 (segment (start 130.563 81.7) (end 133.381 78.882) (width 0.8) (layer "B.Cu") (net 21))
 (segment (start 103.73 76.681) (end 108.749 81.7) (width 0.8) (layer "B.Cu") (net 21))
 (segment (start 108.749 81.7) (end 130.563 81.7) (width 0.8) (layer "B.Cu") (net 21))
 (segment (start 105.48 72.621) (end 103.73 74.371) (width 0.8) (layer "B.Cu") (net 21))
 (segment (start 133.381 74.882) (end 129.851 71.352) (width 0.8) (layer "B.Cu") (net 21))
 (segment (start 103.73 74.371) (end 103.73 76.681) (width 0.8) (layer "B.Cu") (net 21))
 (segment (start 133.381 78.882) (end 133.381 74.882) (width 0.8) (layer "B.Cu") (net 21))
 (segment (start 129.851 71.352) (end 124.521 71.352) (width 0.8) (layer "B.Cu") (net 21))
 (segment (start 108.351 71.682) (end 108.02 71.351) (width 0.8) (layer "F.Cu") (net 20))
 (segment (start 114.132 69.30876) (end 114.132 69.281) (width 0.8) (layer "F.Cu") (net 20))
 (segment (start 111.731 71.682) (end 108.351 71.682) (width 0.8) (layer "F.Cu") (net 20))
 (segment (start 114.132 69.281) (end 115.031 68.382) (width 0.8) (layer "F.Cu") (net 20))
 (segment (start 116.481 68.382) (end 116.531 68.432) (width 0.8) (layer "F.Cu") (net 20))
 (segment (start 115.031 68.382) (end 116.481 68.382) (width 0.8) (layer "F.Cu") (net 20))
 (segment (start 113.43 69.983) (end 113.45776 69.983) (width 0.8) (layer "F.Cu") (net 20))
 (segment (start 111.731 71.682) (end 113.43 69.983) (width 0.8) (layer "F.Cu") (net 20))
 (segment (start 113.45776 69.983) (end 114.132 69.30876) (width 0.8) (layer "F.Cu") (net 20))
 (via (at 116.531 68.432) (size 1) (drill 0.4) (layers "F.Cu" "B.Cu") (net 20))
 (segment (start 116.531 68.432) (end 120.721 72.622) (width 0.8) (layer "B.Cu") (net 20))
 (segment (start 120.721 72.622) (end 121.981 72.622) (width 0.8) (layer "B.Cu") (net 20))
 (segment (start 108.04 68.831) (end 108.02 68.811) (width 0.8) (layer "F.Cu") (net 18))
 (segment (start 111.581 67.432) (end 110.531 67.432) (width 0.8) (layer "F.Cu") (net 18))
 (segment (start 110.531 67.432) (end 109.152 68.811) (width 0.8) (layer "F.Cu") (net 18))
 (segment (start 109.152 68.811) (end 108.02 68.811) (width 0.8) (layer "F.Cu") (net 18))
 (segment (start 112.581 68.432) (end 111.581 67.432) (width 0.8) (layer "F.Cu") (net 18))
 (via (at 112.581 68.432) (size 1) (drill 0.4) (layers "F.Cu" "B.Cu") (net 18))
 (segment (start 119.311 75.162) (end 121.981 75.162) (width 0.8) (layer "B.Cu") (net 18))
 (segment (start 112.581 68.432) (end 119.311 75.162) (width 0.8) (layer "B.Cu") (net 18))
 (segment (start 108.581 66.782) (end 118.512 76.713) (width 0.8) (layer "B.Cu") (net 17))
 (segment (start 106.239 66.782) (end 105.48 67.541) (width 0.8) (layer "B.Cu") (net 17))
 (segment (start 124.24 76.713) (end 124.521 76.432) (width 0.8) (layer "B.Cu") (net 17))
 (segment (start 108.581 66.782) (end 106.239 66.782) (width 0.8) (layer "B.Cu") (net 17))
 (segment (start 105.48 67.541) (end 106.24 66.781) (width 0.8) (layer "B.Cu") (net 17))
 (segment (start 118.512 76.713) (end 124.24 76.713) (width 0.8) (layer "B.Cu") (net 17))
 (segment (start 103.53 66.389) (end 103.53 68.693) (width 0.8) (layer "F.Cu") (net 19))
 (segment (start 126.431 72.282) (end 126.431 67.982) (width 0.8) (layer "F.Cu") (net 19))
 (segment (start 124.521 73.892) (end 124.821 73.892) (width 0.8) (layer "F.Cu") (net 19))
 (segment (start 126.431 67.982) (end 123.931 65.482) (width 0.8) (layer "F.Cu") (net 19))
 (segment (start 124.821 73.892) (end 126.431 72.282) (width 0.8) (layer "F.Cu") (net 19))
 (segment (start 104.918 70.081) (end 105.48 70.081) (width 0.8) (layer "F.Cu") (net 19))
 (segment (start 104.439 65.482) (end 104.438 65.481) (width 0.8) (layer "F.Cu") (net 19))
 (segment (start 104.438 65.481) (end 103.53 66.389) (width 0.8) (layer "F.Cu") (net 19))
 (segment (start 123.931 65.482) (end 104.439 65.482) (width 0.8) (layer "F.Cu") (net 19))
 (segment (start 103.53 68.693) (end 104.918 70.081) (width 0.8) (layer "F.Cu") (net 19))
 (segment (start 128.631 69.932) (end 128.631 75.424) (width 0.8) (layer "F.Cu") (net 23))
 (segment (start 125.822 78.231) (end 125.823 78.232) (width 0.8) (layer "F.Cu") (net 23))
 (segment (start 128.631 75.424) (end 125.823 78.232) (width 0.8) (layer "F.Cu") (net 23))
 (segment (start 105.48 76.631) (end 105.48 75.161) (width 0.8) (layer "F.Cu") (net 23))
 (segment (start 107.08 78.231) (end 125.822 78.231) (width 0.8) (layer "F.Cu") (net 23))
 (segment (start 107.08 78.231) (end 105.48 76.631) (width 0.8) (layer "F.Cu") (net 23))
 (via (at 128.631 69.932) (size 1) (drill 0.4) (layers "F.Cu" "B.Cu") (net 23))
 (segment (start 128.631 69.932) (end 127.531 68.832) (width 0.8) (layer "B.Cu") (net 23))
 (segment (start 127.531 68.832) (end 124.541 68.832) (width 0.8) (layer "B.Cu") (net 23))
 (segment (start 124.541 68.832) (end 124.521 68.812) (width 0.8) (layer "B.Cu") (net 23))
 (segment (start 106.258 87.35) (end 105.499 88.109) (width 0.8) (layer "B.Cu") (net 9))
 (segment (start 124.259 97.281) (end 124.54 97) (width 0.8) (layer "B.Cu") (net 9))
 (segment (start 108.6 87.35) (end 118.531 97.281) (width 0.8) (layer "B.Cu") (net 9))
 (segment (start 105.499 88.109) (end 106.259 87.349) (width 0.8) (layer "B.Cu") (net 9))
 (segment (start 108.6 87.35) (end 106.258 87.35) (width 0.8) (layer "B.Cu") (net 9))
 (segment (start 118.531 97.281) (end 124.259 97.281) (width 0.8) (layer "B.Cu") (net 9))
 (segment (start 113.14 94.46) (end 118.85 88.75) (width 0.8) (layer "F.Cu") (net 14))
 (segment (start 113.14 94.46) (end 113.139 94.459) (width 0.8) (layer "F.Cu") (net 14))
 (segment (start 113.139 94.459) (end 108.039 94.459) (width 0.8) (layer "F.Cu") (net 14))
 (via (at 118.85 88.75) (size 1) (drill 0.4) (layers "F.Cu" "B.Cu") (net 14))
 (segment (start 118.85 88.75) (end 120.1 88.75) (width 0.8) (layer "B.Cu") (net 14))
 (segment (start 120.1 88.75) (end 122 90.65) (width 0.8) (layer "B.Cu") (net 14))
 (segment (start 110.55 88) (end 109.171 89.379) (width 0.8) (layer "F.Cu") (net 10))
 (segment (start 112.6 89) (end 111.6 88) (width 0.8) (layer "F.Cu") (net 10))
 (segment (start 111.6 88) (end 110.55 88) (width 0.8) (layer "F.Cu") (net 10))
 (segment (start 109.171 89.379) (end 108.039 89.379) (width 0.8) (layer "F.Cu") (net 10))
 (segment (start 108.059 89.399) (end 108.039 89.379) (width 0.8) (layer "F.Cu") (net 10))
 (via (at 112.6 89) (size 1) (drill 0.4) (layers "F.Cu" "B.Cu") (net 10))
 (segment (start 119.33 95.73) (end 122 95.73) (width 0.8) (layer "B.Cu") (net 10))
 (segment (start 112.6 89) (end 119.33 95.73) (width 0.8) (layer "B.Cu") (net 10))
 (segment (start 133.4 99.45) (end 133.4 95.45) (width 0.8) (layer "B.Cu") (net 13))
 (segment (start 108.8 102.3) (end 130.55 102.3) (width 0.8) (layer "B.Cu") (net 13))
 (segment (start 130.55 102.3) (end 133.4 99.45) (width 0.8) (layer "B.Cu") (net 13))
 (segment (start 103.749 97.249) (end 108.8 102.3) (width 0.8) (layer "B.Cu") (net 13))
 (segment (start 129.87 91.92) (end 124.54 91.92) (width 0.8) (layer "B.Cu") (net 13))
 (segment (start 105.499 93.189) (end 103.749 94.939) (width 0.8) (layer "B.Cu") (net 13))
 (segment (start 133.4 95.45) (end 129.87 91.92) (width 0.8) (layer "B.Cu") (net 13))
 (segment (start 103.749 94.939) (end 103.749 97.249) (width 0.8) (layer "B.Cu") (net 13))
 (segment (start 103.549 89.261) (end 104.937 90.649) (width 0.8) (layer "F.Cu") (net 11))
 (segment (start 103.549 86.957) (end 103.549 89.261) (width 0.8) (layer "F.Cu") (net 11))
 (segment (start 126.45 92.85) (end 126.45 88.55) (width 0.8) (layer "F.Cu") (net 11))
 (segment (start 124.54 94.46) (end 124.84 94.46) (width 0.8) (layer "F.Cu") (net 11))
 (segment (start 123.95 86.05) (end 104.458 86.05) (width 0.8) (layer "F.Cu") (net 11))
 (segment (start 104.458 86.05) (end 104.457 86.049) (width 0.8) (layer "F.Cu") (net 11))
 (segment (start 124.84 94.46) (end 126.45 92.85) (width 0.8) (layer "F.Cu") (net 11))
 (segment (start 104.937 90.649) (end 105.499 90.649) (width 0.8) (layer "F.Cu") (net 11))
 (segment (start 126.45 88.55) (end 123.95 86.05) (width 0.8) (layer "F.Cu") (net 11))
 (segment (start 104.457 86.049) (end 103.549 86.957) (width 0.8) (layer "F.Cu") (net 11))
 (segment (start 107.099 98.799) (end 125.841 98.799) (width 0.8) (layer "F.Cu") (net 15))
 (segment (start 125.841 98.799) (end 125.842 98.8) (width 0.8) (layer "F.Cu") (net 15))
 (segment (start 128.65 95.992) (end 125.842 98.8) (width 0.8) (layer "F.Cu") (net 15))
 (segment (start 107.099 98.799) (end 105.499 97.199) (width 0.8) (layer "F.Cu") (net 15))
 (segment (start 105.499 97.199) (end 105.499 95.729) (width 0.8) (layer "F.Cu") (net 15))
 (segment (start 128.65 90.5) (end 128.65 95.992) (width 0.8) (layer "F.Cu") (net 15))
 (via (at 128.65 90.5) (size 1) (drill 0.4) (layers "F.Cu" "B.Cu") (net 15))
 (segment (start 128.65 90.5) (end 127.55 89.4) (width 0.8) (layer "B.Cu") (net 15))
 (segment (start 124.56 89.4) (end 124.54 89.38) (width 0.8) (layer "B.Cu") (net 15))
 (segment (start 127.55 89.4) (end 124.56 89.4) (width 0.8) (layer "B.Cu") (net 15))
 (segment (start 113.11 97) (end 113.109 96.999) (width 0.8) (layer "F.Cu") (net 16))
 (segment (start 113.109 96.999) (end 108.039 96.999) (width 0.8) (layer "F.Cu") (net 16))
 (segment (start 113.11 97) (end 122 88.11) (width 0.8) (layer "F.Cu") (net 16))
 (segment (start 116.5 88.95) (end 116.55 89) (width 0.8) (layer "F.Cu") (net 12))
 (segment (start 111.75 92.25) (end 113.449 90.551) (width 0.8) (layer "F.Cu") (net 12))
 (segment (start 114.151 89.849) (end 115.05 88.95) (width 0.8) (layer "F.Cu") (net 12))
 (segment (start 108.37 92.25) (end 108.039 91.919) (width 0.8) (layer "F.Cu") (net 12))
 (segment (start 113.47676 90.551) (end 114.151 89.87676) (width 0.8) (layer "F.Cu") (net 12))
 (segment (start 114.151 89.87676) (end 114.151 89.849) (width 0.8) (layer "F.Cu") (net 12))
 (segment (start 111.75 92.25) (end 108.37 92.25) (width 0.8) (layer "F.Cu") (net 12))
 (segment (start 113.449 90.551) (end 113.47676 90.551) (width 0.8) (layer "F.Cu") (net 12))
 (segment (start 115.05 88.95) (end 116.5 88.95) (width 0.8) (layer "F.Cu") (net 12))
 (via (at 116.55 89) (size 1) (drill 0.4) (layers "F.Cu" "B.Cu") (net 12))
 (segment (start 116.55 89) (end 120.74 93.19) (width 0.8) (layer "B.Cu") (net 12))
 (segment (start 120.74 93.19) (end 122 93.19) (width 0.8) (layer "B.Cu") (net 12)))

